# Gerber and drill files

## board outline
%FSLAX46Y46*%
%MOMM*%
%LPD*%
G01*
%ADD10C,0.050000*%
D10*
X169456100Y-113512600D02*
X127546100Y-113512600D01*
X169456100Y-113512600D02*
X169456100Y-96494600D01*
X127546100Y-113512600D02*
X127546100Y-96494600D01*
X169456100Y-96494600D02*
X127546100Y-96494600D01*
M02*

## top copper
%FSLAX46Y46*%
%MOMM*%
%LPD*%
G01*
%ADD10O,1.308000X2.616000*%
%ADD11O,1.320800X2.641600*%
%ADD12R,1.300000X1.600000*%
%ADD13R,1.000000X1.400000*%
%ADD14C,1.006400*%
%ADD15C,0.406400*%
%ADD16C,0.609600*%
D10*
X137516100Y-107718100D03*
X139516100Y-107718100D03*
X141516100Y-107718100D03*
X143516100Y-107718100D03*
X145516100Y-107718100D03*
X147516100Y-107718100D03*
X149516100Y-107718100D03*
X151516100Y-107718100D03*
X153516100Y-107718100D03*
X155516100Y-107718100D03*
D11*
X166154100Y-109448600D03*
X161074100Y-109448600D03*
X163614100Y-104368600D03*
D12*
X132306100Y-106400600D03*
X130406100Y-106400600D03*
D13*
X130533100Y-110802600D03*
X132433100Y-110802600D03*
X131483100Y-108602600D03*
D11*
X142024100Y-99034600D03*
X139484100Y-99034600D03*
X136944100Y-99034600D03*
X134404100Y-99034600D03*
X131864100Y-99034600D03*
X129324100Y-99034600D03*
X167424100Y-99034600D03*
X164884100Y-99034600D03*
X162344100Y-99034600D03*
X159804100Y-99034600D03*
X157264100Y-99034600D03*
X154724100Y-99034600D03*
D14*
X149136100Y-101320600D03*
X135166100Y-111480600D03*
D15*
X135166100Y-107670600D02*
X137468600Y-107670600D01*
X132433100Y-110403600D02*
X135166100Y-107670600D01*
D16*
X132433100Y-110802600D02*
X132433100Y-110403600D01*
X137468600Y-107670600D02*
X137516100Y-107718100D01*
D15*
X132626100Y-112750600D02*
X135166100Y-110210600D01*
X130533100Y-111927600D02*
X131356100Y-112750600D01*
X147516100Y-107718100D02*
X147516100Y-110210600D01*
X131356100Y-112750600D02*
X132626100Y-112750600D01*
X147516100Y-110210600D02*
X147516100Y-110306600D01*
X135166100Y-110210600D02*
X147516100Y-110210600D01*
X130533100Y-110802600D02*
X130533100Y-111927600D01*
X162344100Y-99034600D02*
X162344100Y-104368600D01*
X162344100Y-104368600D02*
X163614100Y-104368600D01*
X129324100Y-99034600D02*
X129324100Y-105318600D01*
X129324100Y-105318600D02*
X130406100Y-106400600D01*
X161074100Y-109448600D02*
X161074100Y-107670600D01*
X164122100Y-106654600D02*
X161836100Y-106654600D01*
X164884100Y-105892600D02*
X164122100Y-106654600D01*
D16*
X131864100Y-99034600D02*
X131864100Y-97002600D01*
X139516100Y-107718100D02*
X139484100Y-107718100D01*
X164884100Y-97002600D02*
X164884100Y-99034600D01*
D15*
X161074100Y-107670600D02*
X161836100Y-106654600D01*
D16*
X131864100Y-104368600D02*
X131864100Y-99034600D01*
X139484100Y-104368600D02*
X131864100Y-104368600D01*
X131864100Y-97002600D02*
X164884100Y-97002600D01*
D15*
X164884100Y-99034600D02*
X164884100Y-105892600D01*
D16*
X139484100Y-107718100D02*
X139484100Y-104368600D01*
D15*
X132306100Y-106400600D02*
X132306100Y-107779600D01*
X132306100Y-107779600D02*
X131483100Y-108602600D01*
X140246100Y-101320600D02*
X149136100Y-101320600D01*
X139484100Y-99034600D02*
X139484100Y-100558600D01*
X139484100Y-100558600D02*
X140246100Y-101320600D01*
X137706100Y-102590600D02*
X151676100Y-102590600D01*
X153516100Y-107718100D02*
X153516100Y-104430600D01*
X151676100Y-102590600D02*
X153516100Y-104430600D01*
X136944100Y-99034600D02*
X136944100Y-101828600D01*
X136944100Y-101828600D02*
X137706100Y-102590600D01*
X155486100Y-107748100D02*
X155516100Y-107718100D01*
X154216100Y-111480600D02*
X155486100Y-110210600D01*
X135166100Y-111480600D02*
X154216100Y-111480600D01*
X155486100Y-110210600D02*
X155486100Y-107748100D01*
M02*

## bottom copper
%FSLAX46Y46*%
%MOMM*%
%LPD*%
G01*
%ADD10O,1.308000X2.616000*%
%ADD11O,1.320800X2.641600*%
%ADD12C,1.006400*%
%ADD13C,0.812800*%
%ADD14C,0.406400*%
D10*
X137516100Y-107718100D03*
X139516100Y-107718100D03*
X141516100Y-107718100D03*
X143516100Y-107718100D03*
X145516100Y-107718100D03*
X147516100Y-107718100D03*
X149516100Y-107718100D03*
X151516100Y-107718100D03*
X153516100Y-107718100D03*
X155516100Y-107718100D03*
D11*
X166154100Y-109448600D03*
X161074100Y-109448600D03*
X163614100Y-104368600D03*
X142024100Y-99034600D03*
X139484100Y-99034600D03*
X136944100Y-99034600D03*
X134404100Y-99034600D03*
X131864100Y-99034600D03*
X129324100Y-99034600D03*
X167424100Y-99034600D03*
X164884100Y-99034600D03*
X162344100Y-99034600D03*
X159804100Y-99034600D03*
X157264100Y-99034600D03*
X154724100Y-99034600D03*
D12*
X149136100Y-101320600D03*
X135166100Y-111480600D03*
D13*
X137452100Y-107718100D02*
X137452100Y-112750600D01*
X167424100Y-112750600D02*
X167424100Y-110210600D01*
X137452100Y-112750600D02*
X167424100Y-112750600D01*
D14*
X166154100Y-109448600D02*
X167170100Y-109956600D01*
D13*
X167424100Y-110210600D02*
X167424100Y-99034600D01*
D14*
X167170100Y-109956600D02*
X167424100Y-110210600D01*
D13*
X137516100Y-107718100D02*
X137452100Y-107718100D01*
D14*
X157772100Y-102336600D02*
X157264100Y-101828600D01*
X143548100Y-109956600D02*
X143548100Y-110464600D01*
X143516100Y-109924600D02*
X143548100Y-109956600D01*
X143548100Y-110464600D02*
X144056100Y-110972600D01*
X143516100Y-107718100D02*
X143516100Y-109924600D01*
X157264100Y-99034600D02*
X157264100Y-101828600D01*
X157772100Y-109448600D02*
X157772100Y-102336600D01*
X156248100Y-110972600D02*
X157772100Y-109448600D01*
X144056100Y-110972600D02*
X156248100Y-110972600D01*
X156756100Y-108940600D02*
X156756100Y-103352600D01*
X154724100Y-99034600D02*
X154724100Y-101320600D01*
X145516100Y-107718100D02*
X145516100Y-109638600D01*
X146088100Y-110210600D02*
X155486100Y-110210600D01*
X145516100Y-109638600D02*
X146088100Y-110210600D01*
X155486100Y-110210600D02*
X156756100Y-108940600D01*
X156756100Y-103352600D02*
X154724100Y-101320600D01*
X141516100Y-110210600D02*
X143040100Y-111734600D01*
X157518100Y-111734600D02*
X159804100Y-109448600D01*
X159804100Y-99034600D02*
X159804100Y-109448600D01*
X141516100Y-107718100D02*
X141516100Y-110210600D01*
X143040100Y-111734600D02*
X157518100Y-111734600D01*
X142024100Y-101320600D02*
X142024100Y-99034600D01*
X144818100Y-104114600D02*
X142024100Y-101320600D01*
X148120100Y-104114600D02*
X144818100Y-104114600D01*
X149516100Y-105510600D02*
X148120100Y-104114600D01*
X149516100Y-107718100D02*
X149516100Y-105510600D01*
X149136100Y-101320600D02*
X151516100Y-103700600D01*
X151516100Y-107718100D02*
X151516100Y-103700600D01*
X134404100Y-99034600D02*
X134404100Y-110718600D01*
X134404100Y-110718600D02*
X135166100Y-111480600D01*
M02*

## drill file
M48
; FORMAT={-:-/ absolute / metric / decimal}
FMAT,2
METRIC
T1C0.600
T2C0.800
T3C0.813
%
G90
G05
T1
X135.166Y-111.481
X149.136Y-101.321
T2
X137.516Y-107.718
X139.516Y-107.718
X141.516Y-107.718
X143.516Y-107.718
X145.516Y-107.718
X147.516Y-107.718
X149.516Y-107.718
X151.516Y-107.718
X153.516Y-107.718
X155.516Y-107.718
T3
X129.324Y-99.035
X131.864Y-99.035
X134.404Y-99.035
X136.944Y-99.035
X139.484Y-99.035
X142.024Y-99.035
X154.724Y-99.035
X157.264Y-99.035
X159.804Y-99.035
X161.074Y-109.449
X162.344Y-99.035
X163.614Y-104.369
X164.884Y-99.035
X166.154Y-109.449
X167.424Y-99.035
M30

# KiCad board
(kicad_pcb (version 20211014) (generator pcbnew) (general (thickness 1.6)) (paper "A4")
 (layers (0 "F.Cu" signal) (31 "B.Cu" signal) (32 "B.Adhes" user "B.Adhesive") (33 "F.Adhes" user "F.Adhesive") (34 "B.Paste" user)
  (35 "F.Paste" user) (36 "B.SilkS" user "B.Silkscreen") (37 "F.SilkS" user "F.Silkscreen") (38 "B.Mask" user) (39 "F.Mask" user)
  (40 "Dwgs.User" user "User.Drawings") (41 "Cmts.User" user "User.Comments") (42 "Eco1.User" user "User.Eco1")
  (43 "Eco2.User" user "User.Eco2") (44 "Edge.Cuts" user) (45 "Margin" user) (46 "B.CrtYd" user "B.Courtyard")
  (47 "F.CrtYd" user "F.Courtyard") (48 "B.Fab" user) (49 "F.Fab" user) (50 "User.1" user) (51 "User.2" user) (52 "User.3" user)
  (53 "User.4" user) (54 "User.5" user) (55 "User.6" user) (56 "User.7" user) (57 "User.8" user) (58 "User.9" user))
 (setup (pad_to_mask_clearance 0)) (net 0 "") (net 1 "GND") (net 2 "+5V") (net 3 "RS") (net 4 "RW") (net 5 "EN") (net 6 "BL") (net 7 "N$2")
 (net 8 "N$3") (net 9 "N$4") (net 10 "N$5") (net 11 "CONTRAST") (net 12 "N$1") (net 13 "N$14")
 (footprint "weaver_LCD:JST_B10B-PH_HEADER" (layer "F.Cu") (at 141.5161 107.6706 180)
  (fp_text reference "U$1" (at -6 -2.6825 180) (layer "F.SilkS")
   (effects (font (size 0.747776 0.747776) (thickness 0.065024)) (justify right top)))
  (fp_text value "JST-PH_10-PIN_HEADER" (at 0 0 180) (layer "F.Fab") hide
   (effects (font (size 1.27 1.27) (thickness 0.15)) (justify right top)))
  (pad "P1" thru_hole oval (at 4 -0.0475 270) (size 2.616 1.308) (drill 0.8) (layers *.Cu *.Mask) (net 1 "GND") (solder_mask_margin 0.1016))
  (pad "P2" thru_hole oval (at 2 -0.0475 270) (size 2.616 1.308) (drill 0.8) (layers *.Cu *.Mask) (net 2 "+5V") (solder_mask_margin 0.1016))
  (pad "P3" thru_hole oval (at 0 -0.0475 270) (size 2.616 1.308) (drill 0.8) (layers *.Cu *.Mask) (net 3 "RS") (solder_mask_margin 0.1016))
  (pad "P4" thru_hole oval (at -2 -0.0475 270) (size 2.616 1.308) (drill 0.8) (layers *.Cu *.Mask) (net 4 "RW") (solder_mask_margin 0.1016))
  (pad "P5" thru_hole oval (at -4 -0.0475 270) (size 2.616 1.308) (drill 0.8) (layers *.Cu *.Mask) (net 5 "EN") (solder_mask_margin 0.1016))
  (pad "P6" thru_hole oval (at -6 -0.0475 270) (size 2.616 1.308) (drill 0.8) (layers *.Cu *.Mask) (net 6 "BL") (solder_mask_margin 0.1016))
  (pad "P7" thru_hole oval (at -8 -0.0475 270) (size 2.616 1.308) (drill 0.8) (layers *.Cu *.Mask) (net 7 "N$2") (solder_mask_margin 0.1016))
  (pad "P8" thru_hole oval (at -10 -0.0475 270) (size 2.616 1.308) (drill 0.8) (layers *.Cu *.Mask) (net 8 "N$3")
   (solder_mask_margin 0.1016))
  (pad "P9" thru_hole oval (at -12 -0.0475 270) (size 2.616 1.308) (drill 0.8) (layers *.Cu *.Mask) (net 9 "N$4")
   (solder_mask_margin 0.1016))
  (pad "P10" thru_hole oval (at -14 -0.0475 270) (size 2.616 1.308) (drill 0.8) (layers *.Cu *.Mask) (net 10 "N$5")
   (solder_mask_margin 0.1016)))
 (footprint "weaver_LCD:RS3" (layer "F.Cu") (at 163.6141 106.9086 180)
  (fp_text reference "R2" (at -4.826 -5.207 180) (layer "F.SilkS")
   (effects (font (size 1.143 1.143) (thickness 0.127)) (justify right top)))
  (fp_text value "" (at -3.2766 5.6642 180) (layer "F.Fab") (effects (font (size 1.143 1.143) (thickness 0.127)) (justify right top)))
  (pad "A" thru_hole oval (at -2.54 -2.54 270) (size 2.6416 1.3208) (drill 0.8128) (layers *.Cu *.Mask) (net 1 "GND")
   (solder_mask_margin 0.1016))
  (pad "E" thru_hole oval (at 2.54 -2.54 270) (size 2.6416 1.3208) (drill 0.8128) (layers *.Cu *.Mask) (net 2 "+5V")
   (solder_mask_margin 0.1016))
  (pad "S" thru_hole oval (at 0 2.54 270) (size 2.6416 1.3208) (drill 0.8128) (layers *.Cu *.Mask) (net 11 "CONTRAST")
   (solder_mask_margin 0.1016)))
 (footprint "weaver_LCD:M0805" (layer "F.Cu") (at 131.3561 106.4006 180)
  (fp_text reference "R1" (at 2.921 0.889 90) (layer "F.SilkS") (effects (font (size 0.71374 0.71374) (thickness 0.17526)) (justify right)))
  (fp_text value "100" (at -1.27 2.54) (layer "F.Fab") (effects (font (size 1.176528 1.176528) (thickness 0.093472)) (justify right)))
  (pad "1" smd rect (at -0.95 0 180) (size 1.3 1.6) (layers "F.Cu" "F.Paste" "F.Mask") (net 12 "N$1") (solder_mask_margin 0.1016))
  (pad "2" smd rect (at 0.95 0 180) (size 1.3 1.6) (layers "F.Cu" "F.Paste" "F.Mask") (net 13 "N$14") (solder_mask_margin 0.1016)))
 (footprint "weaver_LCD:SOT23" (layer "F.Cu") (at 131.4831 109.7026)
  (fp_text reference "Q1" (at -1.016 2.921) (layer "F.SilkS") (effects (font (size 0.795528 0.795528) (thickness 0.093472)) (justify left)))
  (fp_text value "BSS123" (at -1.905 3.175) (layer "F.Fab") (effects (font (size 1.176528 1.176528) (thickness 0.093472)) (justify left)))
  (pad "1" smd rect (at -0.95 1.1) (size 1 1.4) (layers "F.Cu" "F.Paste" "F.Mask") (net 6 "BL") (solder_mask_margin 0.1016))
  (pad "2" smd rect (at 0.95 1.1) (size 1 1.4) (layers "F.Cu" "F.Paste" "F.Mask") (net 1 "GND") (solder_mask_margin 0.1016))
  (pad "3" smd rect (at 0 -1.1) (size 1 1.4) (layers "F.Cu" "F.Paste" "F.Mask") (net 12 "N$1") (solder_mask_margin 0.1016)))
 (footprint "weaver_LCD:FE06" (layer "B.Cu") (at 135.6741 99.0346 180)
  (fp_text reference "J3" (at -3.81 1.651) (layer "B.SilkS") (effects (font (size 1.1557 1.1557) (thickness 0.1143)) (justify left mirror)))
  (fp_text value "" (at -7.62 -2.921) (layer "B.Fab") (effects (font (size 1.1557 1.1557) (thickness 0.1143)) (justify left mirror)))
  (pad "1" thru_hole oval (at -6.35 0 90) (size 2.6416 1.3208) (drill 0.8128) (layers *.Cu *.Mask) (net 7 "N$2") (solder_mask_margin 0.1016))
  (pad "2" thru_hole oval (at -3.81 0 90) (size 2.6416 1.3208) (drill 0.8128) (layers *.Cu *.Mask) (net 8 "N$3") (solder_mask_margin 0.1016))
  (pad "3" thru_hole oval (at -1.27 0 90) (size 2.6416 1.3208) (drill 0.8128) (layers *.Cu *.Mask) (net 9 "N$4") (solder_mask_margin 0.1016))
  (pad "4" thru_hole oval (at 1.27 0 90) (size 2.6416 1.3208) (drill 0.8128) (layers *.Cu *.Mask) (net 10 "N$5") (solder_mask_margin 0.1016))
  (pad "5" thru_hole oval (at 3.81 0 90) (size 2.6416 1.3208) (drill 0.8128) (layers *.Cu *.Mask) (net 2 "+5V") (solder_mask_margin 0.1016))
  (pad "6" thru_hole oval (at 6.35 0 90) (size 2.6416 1.3208) (drill 0.8128) (layers *.Cu *.Mask) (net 13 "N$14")
   (solder_mask_margin 0.1016)))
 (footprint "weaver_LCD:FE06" (layer "B.Cu") (at 161.0741 99.0346 180)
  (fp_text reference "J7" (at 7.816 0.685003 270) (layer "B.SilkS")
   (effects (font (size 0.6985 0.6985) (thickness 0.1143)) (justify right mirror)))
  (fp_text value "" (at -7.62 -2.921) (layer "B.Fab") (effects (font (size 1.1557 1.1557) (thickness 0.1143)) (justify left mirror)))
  (pad "1" thru_hole oval (at -6.35 0 90) (size 2.6416 1.3208) (drill 0.8128) (layers *.Cu *.Mask) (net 1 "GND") (solder_mask_margin 0.1016))
  (pad "2" thru_hole oval (at -3.81 0 90) (size 2.6416 1.3208) (drill 0.8128) (layers *.Cu *.Mask) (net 2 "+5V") (solder_mask_margin 0.1016))
  (pad "3" thru_hole oval (at -1.27 0 90) (size 2.6416 1.3208) (drill 0.8128) (layers *.Cu *.Mask) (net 11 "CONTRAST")
   (solder_mask_margin 0.1016))
  (pad "4" thru_hole oval (at 1.27 0 90) (size 2.6416 1.3208) (drill 0.8128) (layers *.Cu *.Mask) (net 3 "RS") (solder_mask_margin 0.1016))
  (pad "5" thru_hole oval (at 3.81 0 90) (size 2.6416 1.3208) (drill 0.8128) (layers *.Cu *.Mask) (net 4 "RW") (solder_mask_margin 0.1016))
  (pad "6" thru_hole oval (at 6.35 0 90) (size 2.6416 1.3208) (drill 0.8128) (layers *.Cu *.Mask) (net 5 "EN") (solder_mask_margin 0.1016)))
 (gr_line (start 169.4561 113.5126) (end 127.5461 113.5126) (layer "Edge.Cuts") (width 0.05))
 (gr_line (start 169.4561 113.5126) (end 169.4561 96.4946) (layer "Edge.Cuts") (width 0.05))
 (gr_line (start 127.5461 113.5126) (end 127.5461 96.4946) (layer "Edge.Cuts") (width 0.05))
 (gr_line (start 169.4561 96.4946) (end 127.5461 96.4946) (layer "Edge.Cuts") (width 0.05))
 (segment (start 135.1661 107.6706) (end 137.4686 107.6706) (width 0.4064) (layer "F.Cu") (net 1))
 (segment (start 132.4331 110.4036) (end 135.1661 107.6706) (width 0.4064) (layer "F.Cu") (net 1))
 (segment (start 132.4331 110.8026) (end 132.4331 110.4036) (width 0.6096) (layer "F.Cu") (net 1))
 (segment (start 137.4686 107.6706) (end 137.5161 107.7181) (width 0.6096) (layer "F.Cu") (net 1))
 (segment (start 137.4521 107.7181) (end 137.4521 112.7506) (width 0.8128) (layer "B.Cu") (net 1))
 (segment (start 167.4241 112.7506) (end 167.4241 110.2106) (width 0.8128) (layer "B.Cu") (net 1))
 (segment (start 137.4521 112.7506) (end 167.4241 112.7506) (width 0.8128) (layer "B.Cu") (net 1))
 (segment (start 166.1541 109.4486) (end 167.1701 109.9566) (width 0.4064) (layer "B.Cu") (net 1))
 (segment (start 167.4241 110.2106) (end 167.4241 99.0346) (width 0.8128) (layer "B.Cu") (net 1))
 (segment (start 167.1701 109.9566) (end 167.4241 110.2106) (width 0.4064) (layer "B.Cu") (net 1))
 (segment (start 137.5161 107.7181) (end 137.4521 107.7181) (width 0.8128) (layer "B.Cu") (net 1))
 (segment (start 157.7721 102.3366) (end 157.2641 101.8286) (width 0.4064) (layer "B.Cu") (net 4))
 (segment (start 143.5481 109.9566) (end 143.5481 110.4646) (width 0.4064) (layer "B.Cu") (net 4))
 (segment (start 143.5161 109.9246) (end 143.5481 109.9566) (width 0.4064) (layer "B.Cu") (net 4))
 (segment (start 143.5481 110.4646) (end 144.0561 110.9726) (width 0.4064) (layer "B.Cu") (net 4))
 (segment (start 143.5161 107.7181) (end 143.5161 109.9246) (width 0.4064) (layer "B.Cu") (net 4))
 (segment (start 157.2641 99.0346) (end 157.2641 101.8286) (width 0.4064) (layer "B.Cu") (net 4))
 (segment (start 157.7721 109.4486) (end 157.7721 102.3366) (width 0.4064) (layer "B.Cu") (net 4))
 (segment (start 156.2481 110.9726) (end 157.7721 109.4486) (width 0.4064) (layer "B.Cu") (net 4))
 (segment (start 144.0561 110.9726) (end 156.2481 110.9726) (width 0.4064) (layer "B.Cu") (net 4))
 (segment (start 132.6261 112.7506) (end 135.1661 110.2106) (width 0.4064) (layer "F.Cu") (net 6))
 (segment (start 130.5331 111.9276) (end 131.3561 112.7506) (width 0.4064) (layer "F.Cu") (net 6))
 (segment (start 147.5161 107.7181) (end 147.5161 110.2106) (width 0.4064) (layer "F.Cu") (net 6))
 (segment (start 131.3561 112.7506) (end 132.6261 112.7506) (width 0.4064) (layer "F.Cu") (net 6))
 (segment (start 147.5161 110.2106) (end 147.5161 110.3066) (width 0.4064) (layer "F.Cu") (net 6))
 (segment (start 135.1661 110.2106) (end 147.5161 110.2106) (width 0.4064) (layer "F.Cu") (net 6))
 (segment (start 130.5331 110.8026) (end 130.5331 111.9276) (width 0.4064) (layer "F.Cu") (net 6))
 (segment (start 156.7561 108.9406) (end 156.7561 103.3526) (width 0.4064) (layer "B.Cu") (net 5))
 (segment (start 154.7241 99.0346) (end 154.7241 101.3206) (width 0.4064) (layer "B.Cu") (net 5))
 (segment (start 145.5161 107.7181) (end 145.5161 109.6386) (width 0.4064) (layer "B.Cu") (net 5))
 (segment (start 146.0881 110.2106) (end 155.4861 110.2106) (width 0.4064) (layer "B.Cu") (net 5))
 (segment (start 145.5161 109.6386) (end 146.0881 110.2106) (width 0.4064) (layer "B.Cu") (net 5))
 (segment (start 155.4861 110.2106) (end 156.7561 108.9406) (width 0.4064) (layer "B.Cu") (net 5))
 (segment (start 156.7561 103.3526) (end 154.7241 101.3206) (width 0.4064) (layer "B.Cu") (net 5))
 (segment (start 162.3441 99.0346) (end 162.3441 104.3686) (width 0.4064) (layer "F.Cu") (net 11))
 (segment (start 162.3441 104.3686) (end 163.6141 104.3686) (width 0.4064) (layer "F.Cu") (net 11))
 (segment (start 129.3241 99.0346) (end 129.3241 105.3186) (width 0.4064) (layer "F.Cu") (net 13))
 (segment (start 129.3241 105.3186) (end 130.4061 106.4006) (width 0.4064) (layer "F.Cu") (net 13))
 (segment (start 161.0741 109.4486) (end 161.0741 107.6706) (width 0.4064) (layer "F.Cu") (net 2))
 (segment (start 164.1221 106.6546) (end 161.8361 106.6546) (width 0.4064) (layer "F.Cu") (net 2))
 (segment (start 164.8841 105.8926) (end 164.1221 106.6546) (width 0.4064) (layer "F.Cu") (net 2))
 (segment (start 131.8641 99.0346) (end 131.8641 97.0026) (width 0.6096) (layer "F.Cu") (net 2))
 (segment (start 139.5161 107.7181) (end 139.4841 107.7181) (width 0.6096) (layer "F.Cu") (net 2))
 (segment (start 164.8841 97.0026) (end 164.8841 99.0346) (width 0.6096) (layer "F.Cu") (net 2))
 (segment (start 161.0741 107.6706) (end 161.8361 106.6546) (width 0.4064) (layer "F.Cu") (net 2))
 (segment (start 131.8641 104.3686) (end 131.8641 99.0346) (width 0.6096) (layer "F.Cu") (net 2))
 (segment (start 139.4841 104.3686) (end 131.8641 104.3686) (width 0.6096) (layer "F.Cu") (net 2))
 (segment (start 131.8641 97.0026) (end 164.8841 97.0026) (width 0.6096) (layer "F.Cu") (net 2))
 (segment (start 164.8841 99.0346) (end 164.8841 105.8926) (width 0.4064) (layer "F.Cu") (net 2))
 (segment (start 139.4841 107.7181) (end 139.4841 104.3686) (width 0.6096) (layer "F.Cu") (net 2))
 (segment (start 132.3061 106.4006) (end 132.3061 107.7796) (width 0.4064) (layer "F.Cu") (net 12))
 (segment (start 132.3061 107.7796) (end 131.4831 108.6026) (width 0.4064) (layer "F.Cu") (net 12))
 (segment (start 141.5161 110.2106) (end 143.0401 111.7346) (width 0.4064) (layer "B.Cu") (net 3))
 (segment (start 157.5181 111.7346) (end 159.8041 109.4486) (width 0.4064) (layer "B.Cu") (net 3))
 (segment (start 159.8041 99.0346) (end 159.8041 109.4486) (width 0.4064) (layer "B.Cu") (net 3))
 (segment (start 141.5161 107.7181) (end 141.5161 110.2106) (width 0.4064) (layer "B.Cu") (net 3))
 (segment (start 143.0401 111.7346) (end 157.5181 111.7346) (width 0.4064) (layer "B.Cu") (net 3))
 (segment (start 142.0241 101.3206) (end 142.0241 99.0346) (width 0.4064) (layer "B.Cu") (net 7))
 (segment (start 144.8181 104.1146) (end 142.0241 101.3206) (width 0.4064) (layer "B.Cu") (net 7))
 (segment (start 148.1201 104.1146) (end 144.8181 104.1146) (width 0.4064) (layer "B.Cu") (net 7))
 (segment (start 149.5161 105.5106) (end 148.1201 104.1146) (width 0.4064) (layer "B.Cu") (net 7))
 (segment (start 149.5161 107.7181) (end 149.5161 105.5106) (width 0.4064) (layer "B.Cu") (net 7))
 (segment (start 140.2461 101.3206) (end 149.1361 101.3206) (width 0.4064) (layer "F.Cu") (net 8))
 (segment (start 139.4841 99.0346) (end 139.4841 100.5586) (width 0.4064) (layer "F.Cu") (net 8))
 (segment (start 139.4841 100.5586) (end 140.2461 101.3206) (width 0.4064) (layer "F.Cu") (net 8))
 (via (at 149.1361 101.3206) (size 1.0064) (drill 0.6) (layers "F.Cu" "B.Cu") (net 8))
 (segment (start 149.1361 101.3206) (end 151.5161 103.7006) (width 0.4064) (layer "B.Cu") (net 8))
 (segment (start 151.5161 107.7181) (end 151.5161 103.7006) (width 0.4064) (layer "B.Cu") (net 8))
 (segment (start 137.7061 102.5906) (end 151.6761 102.5906) (width 0.4064) (layer "F.Cu") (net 9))
 (segment (start 153.5161 107.7181) (end 153.5161 104.4306) (width 0.4064) (layer "F.Cu") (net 9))
 (segment (start 151.6761 102.5906) (end 153.5161 104.4306) (width 0.4064) (layer "F.Cu") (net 9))
 (segment (start 136.9441 99.0346) (end 136.9441 101.8286) (width 0.4064) (layer "F.Cu") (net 9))
 (segment (start 136.9441 101.8286) (end 137.7061 102.5906) (width 0.4064) (layer "F.Cu") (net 9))
 (segment (start 155.4861 107.7481) (end 155.5161 107.7181) (width 0.4064) (layer "F.Cu") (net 10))
 (segment (start 154.2161 111.4806) (end 155.4861 110.2106) (width 0.4064) (layer "F.Cu") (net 10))
 (segment (start 135.1661 111.4806) (end 154.2161 111.4806) (width 0.4064) (layer "F.Cu") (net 10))
 (segment (start 155.4861 110.2106) (end 155.4861 107.7481) (width 0.4064) (layer "F.Cu") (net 10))
 (via (at 135.1661 111.4806) (size 1.0064) (drill 0.6) (layers "F.Cu" "B.Cu") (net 10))
 (segment (start 134.4041 99.0346) (end 134.4041 110.7186) (width 0.4064) (layer "B.Cu") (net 10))
 (segment (start 134.4041 110.7186) (end 135.1661 111.4806) (width 0.4064) (layer "B.Cu") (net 10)))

